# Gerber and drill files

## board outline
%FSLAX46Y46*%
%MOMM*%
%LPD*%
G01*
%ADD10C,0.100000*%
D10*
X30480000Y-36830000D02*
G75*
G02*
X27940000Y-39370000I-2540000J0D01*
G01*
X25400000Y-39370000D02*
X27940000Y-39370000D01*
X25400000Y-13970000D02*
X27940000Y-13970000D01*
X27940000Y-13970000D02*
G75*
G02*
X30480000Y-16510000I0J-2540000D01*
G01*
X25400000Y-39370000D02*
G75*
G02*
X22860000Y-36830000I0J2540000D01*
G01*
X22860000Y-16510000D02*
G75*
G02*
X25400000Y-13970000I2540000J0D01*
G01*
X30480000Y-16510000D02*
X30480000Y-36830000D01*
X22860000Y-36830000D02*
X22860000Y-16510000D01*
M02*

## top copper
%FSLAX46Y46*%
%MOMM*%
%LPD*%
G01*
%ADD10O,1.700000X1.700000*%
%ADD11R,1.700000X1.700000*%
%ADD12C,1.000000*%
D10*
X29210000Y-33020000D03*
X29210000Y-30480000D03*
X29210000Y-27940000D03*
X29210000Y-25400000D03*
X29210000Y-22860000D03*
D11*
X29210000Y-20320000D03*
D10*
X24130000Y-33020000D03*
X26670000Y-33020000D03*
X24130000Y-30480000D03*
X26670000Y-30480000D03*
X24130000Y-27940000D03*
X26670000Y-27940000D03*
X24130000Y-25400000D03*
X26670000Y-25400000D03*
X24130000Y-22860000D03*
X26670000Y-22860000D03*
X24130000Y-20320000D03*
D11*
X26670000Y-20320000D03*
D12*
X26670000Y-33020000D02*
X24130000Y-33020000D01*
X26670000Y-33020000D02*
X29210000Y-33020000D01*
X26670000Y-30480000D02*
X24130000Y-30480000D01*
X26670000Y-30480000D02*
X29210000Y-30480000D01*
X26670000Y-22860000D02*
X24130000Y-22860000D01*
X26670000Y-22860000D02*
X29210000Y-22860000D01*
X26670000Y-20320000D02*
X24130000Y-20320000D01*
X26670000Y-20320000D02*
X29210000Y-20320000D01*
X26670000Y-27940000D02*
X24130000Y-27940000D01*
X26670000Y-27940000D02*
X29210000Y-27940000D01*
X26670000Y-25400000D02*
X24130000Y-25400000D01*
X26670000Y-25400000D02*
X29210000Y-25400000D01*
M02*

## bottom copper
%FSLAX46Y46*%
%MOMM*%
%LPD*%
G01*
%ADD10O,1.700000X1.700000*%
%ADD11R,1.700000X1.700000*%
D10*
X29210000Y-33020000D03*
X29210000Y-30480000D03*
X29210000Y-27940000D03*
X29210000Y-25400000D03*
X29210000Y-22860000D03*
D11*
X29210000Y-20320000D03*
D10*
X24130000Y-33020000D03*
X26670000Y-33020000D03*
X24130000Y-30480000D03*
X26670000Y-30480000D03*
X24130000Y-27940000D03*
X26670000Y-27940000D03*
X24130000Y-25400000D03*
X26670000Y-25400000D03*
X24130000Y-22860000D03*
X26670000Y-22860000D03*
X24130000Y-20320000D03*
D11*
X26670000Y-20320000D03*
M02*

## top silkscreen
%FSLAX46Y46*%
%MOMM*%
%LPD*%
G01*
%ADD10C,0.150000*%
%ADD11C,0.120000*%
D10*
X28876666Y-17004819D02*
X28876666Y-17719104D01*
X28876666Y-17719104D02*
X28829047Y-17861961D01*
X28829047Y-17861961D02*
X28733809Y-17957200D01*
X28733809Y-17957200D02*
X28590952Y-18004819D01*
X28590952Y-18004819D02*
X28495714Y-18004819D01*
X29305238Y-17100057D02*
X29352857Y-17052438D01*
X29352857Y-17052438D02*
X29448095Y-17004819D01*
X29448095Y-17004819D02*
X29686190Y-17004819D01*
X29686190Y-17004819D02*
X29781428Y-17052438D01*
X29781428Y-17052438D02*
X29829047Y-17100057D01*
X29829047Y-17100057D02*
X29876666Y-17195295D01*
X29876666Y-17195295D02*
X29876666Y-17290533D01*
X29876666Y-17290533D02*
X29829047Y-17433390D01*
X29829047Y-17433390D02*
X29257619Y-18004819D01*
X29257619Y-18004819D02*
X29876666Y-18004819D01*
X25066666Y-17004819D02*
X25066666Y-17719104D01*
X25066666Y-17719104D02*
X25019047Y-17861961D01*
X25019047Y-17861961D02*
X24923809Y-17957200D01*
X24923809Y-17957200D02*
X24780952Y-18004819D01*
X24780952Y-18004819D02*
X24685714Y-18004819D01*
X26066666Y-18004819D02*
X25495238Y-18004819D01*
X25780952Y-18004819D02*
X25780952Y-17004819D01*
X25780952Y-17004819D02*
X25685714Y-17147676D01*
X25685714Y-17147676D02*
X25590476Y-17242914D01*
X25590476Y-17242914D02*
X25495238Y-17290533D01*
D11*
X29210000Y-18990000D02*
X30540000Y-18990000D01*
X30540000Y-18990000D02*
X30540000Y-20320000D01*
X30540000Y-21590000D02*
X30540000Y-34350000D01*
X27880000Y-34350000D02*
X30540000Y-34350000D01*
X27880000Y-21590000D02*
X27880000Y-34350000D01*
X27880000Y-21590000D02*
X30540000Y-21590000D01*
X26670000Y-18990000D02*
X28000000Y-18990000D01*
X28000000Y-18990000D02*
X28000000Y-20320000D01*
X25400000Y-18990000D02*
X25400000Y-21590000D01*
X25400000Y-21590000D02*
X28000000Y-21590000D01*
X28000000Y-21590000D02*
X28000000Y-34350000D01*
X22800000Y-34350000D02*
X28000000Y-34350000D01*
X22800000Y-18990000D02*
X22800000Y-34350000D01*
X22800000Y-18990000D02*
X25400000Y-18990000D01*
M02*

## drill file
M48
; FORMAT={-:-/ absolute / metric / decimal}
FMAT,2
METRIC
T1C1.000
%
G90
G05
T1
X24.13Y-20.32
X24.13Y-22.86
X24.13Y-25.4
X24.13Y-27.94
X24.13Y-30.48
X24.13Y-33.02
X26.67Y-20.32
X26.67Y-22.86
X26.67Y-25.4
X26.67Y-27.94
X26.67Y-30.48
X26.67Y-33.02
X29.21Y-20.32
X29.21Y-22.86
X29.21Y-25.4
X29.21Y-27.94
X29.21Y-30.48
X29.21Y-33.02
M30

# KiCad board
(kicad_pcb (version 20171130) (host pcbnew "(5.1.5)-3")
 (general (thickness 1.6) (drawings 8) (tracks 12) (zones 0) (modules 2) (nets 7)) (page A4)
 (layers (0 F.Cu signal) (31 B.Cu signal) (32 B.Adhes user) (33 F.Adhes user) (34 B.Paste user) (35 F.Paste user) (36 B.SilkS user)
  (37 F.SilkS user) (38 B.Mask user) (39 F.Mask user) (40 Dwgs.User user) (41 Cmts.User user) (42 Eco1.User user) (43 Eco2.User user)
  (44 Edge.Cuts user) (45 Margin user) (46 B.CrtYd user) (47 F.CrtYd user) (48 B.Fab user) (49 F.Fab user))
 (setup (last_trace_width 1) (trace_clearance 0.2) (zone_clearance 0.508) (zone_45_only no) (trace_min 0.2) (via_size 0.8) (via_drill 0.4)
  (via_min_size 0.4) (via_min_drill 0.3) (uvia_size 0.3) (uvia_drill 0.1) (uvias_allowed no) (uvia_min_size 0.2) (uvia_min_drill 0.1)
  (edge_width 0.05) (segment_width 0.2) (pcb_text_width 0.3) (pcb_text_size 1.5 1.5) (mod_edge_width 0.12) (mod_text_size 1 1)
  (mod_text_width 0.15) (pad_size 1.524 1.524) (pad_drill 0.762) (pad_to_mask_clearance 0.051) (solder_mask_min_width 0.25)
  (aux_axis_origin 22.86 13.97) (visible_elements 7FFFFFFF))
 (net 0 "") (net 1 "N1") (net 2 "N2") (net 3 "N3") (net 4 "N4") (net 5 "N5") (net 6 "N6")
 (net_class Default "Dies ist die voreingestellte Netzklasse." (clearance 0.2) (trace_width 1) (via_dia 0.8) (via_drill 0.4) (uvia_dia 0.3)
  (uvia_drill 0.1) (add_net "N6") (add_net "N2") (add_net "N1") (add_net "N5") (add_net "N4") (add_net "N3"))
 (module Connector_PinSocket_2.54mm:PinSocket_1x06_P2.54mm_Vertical (layer F.Cu) (at 29.21 20.32)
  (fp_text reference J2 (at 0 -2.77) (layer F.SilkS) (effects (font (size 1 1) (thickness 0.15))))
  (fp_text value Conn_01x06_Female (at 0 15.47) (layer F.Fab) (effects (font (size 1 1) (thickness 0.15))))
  (fp_line (start 0 -1.33) (end 1.33 -1.33) (layer F.SilkS) (width 0.12))
  (fp_line (start 1.33 -1.33) (end 1.33 0) (layer F.SilkS) (width 0.12))
  (fp_line (start 1.33 1.27) (end 1.33 14.03) (layer F.SilkS) (width 0.12))
  (fp_line (start -1.33 14.03) (end 1.33 14.03) (layer F.SilkS) (width 0.12))
  (fp_line (start -1.33 1.27) (end -1.33 14.03) (layer F.SilkS) (width 0.12))
  (fp_line (start -1.33 1.27) (end 1.33 1.27) (layer F.SilkS) (width 0.12))
  (pad 6 thru_hole oval (at 0 12.7) (size 1.7 1.7) (drill 1) (layers *.Cu *.Mask) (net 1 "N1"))
  (pad 5 thru_hole oval (at 0 10.16) (size 1.7 1.7) (drill 1) (layers *.Cu *.Mask) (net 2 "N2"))
  (pad 4 thru_hole oval (at 0 7.62) (size 1.7 1.7) (drill 1) (layers *.Cu *.Mask) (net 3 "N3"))
  (pad 3 thru_hole oval (at 0 5.08) (size 1.7 1.7) (drill 1) (layers *.Cu *.Mask) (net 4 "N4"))
  (pad 2 thru_hole oval (at 0 2.54) (size 1.7 1.7) (drill 1) (layers *.Cu *.Mask) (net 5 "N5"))
  (pad 1 thru_hole rect (at 0 0) (size 1.7 1.7) (drill 1) (layers *.Cu *.Mask) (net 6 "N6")))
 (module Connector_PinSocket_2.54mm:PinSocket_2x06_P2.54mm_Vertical (layer F.Cu) (at 26.67 20.32)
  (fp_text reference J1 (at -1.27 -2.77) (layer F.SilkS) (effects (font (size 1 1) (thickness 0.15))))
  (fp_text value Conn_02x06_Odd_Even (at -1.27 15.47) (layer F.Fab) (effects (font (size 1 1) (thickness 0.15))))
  (fp_line (start 0 -1.33) (end 1.33 -1.33) (layer F.SilkS) (width 0.12))
  (fp_line (start 1.33 -1.33) (end 1.33 0) (layer F.SilkS) (width 0.12))
  (fp_line (start -1.27 -1.33) (end -1.27 1.27) (layer F.SilkS) (width 0.12))
  (fp_line (start -1.27 1.27) (end 1.33 1.27) (layer F.SilkS) (width 0.12))
  (fp_line (start 1.33 1.27) (end 1.33 14.03) (layer F.SilkS) (width 0.12))
  (fp_line (start -3.87 14.03) (end 1.33 14.03) (layer F.SilkS) (width 0.12))
  (fp_line (start -3.87 -1.33) (end -3.87 14.03) (layer F.SilkS) (width 0.12))
  (fp_line (start -3.87 -1.33) (end -1.27 -1.33) (layer F.SilkS) (width 0.12))
  (pad 12 thru_hole oval (at -2.54 12.7) (size 1.7 1.7) (drill 1) (layers *.Cu *.Mask) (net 1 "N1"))
  (pad 11 thru_hole oval (at 0 12.7) (size 1.7 1.7) (drill 1) (layers *.Cu *.Mask) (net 1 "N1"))
  (pad 10 thru_hole oval (at -2.54 10.16) (size 1.7 1.7) (drill 1) (layers *.Cu *.Mask) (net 2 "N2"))
  (pad 9 thru_hole oval (at 0 10.16) (size 1.7 1.7) (drill 1) (layers *.Cu *.Mask) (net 2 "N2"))
  (pad 8 thru_hole oval (at -2.54 7.62) (size 1.7 1.7) (drill 1) (layers *.Cu *.Mask) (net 3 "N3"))
  (pad 7 thru_hole oval (at 0 7.62) (size 1.7 1.7) (drill 1) (layers *.Cu *.Mask) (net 3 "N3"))
  (pad 6 thru_hole oval (at -2.54 5.08) (size 1.7 1.7) (drill 1) (layers *.Cu *.Mask) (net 4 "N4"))
  (pad 5 thru_hole oval (at 0 5.08) (size 1.7 1.7) (drill 1) (layers *.Cu *.Mask) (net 4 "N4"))
  (pad 4 thru_hole oval (at -2.54 2.54) (size 1.7 1.7) (drill 1) (layers *.Cu *.Mask) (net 5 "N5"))
  (pad 3 thru_hole oval (at 0 2.54) (size 1.7 1.7) (drill 1) (layers *.Cu *.Mask) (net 5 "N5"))
  (pad 2 thru_hole oval (at -2.54 0) (size 1.7 1.7) (drill 1) (layers *.Cu *.Mask) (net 6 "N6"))
  (pad 1 thru_hole rect (at 0 0) (size 1.7 1.7) (drill 1) (layers *.Cu *.Mask) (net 6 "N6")))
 (gr_arc (start 27.94 36.83) (end 27.94 39.37) (angle -90) (layer Edge.Cuts) (width 0.1))
 (gr_line (start 25.4 39.37) (end 27.94 39.37) (layer Edge.Cuts) (width 0.1))
 (gr_line (start 25.4 13.97) (end 27.94 13.97) (layer Edge.Cuts) (width 0.1))
 (gr_arc (start 27.94 16.51) (end 30.48 16.51) (angle -90) (layer Edge.Cuts) (width 0.1))
 (gr_arc (start 25.4 36.83) (end 22.86 36.83) (angle -90) (layer Edge.Cuts) (width 0.1))
 (gr_arc (start 25.4 16.51) (end 25.4 13.97) (angle -90) (layer Edge.Cuts) (width 0.1))
 (gr_line (start 30.48 16.51) (end 30.48 36.83) (layer Edge.Cuts) (width 0.1))
 (gr_line (start 22.86 36.83) (end 22.86 16.51) (layer Edge.Cuts) (width 0.1))
 (segment (start 26.67 33.02) (end 24.13 33.02) (width 1) (layer F.Cu) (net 1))
 (segment (start 26.67 33.02) (end 29.21 33.02) (width 1) (layer F.Cu) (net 1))
 (segment (start 26.67 30.48) (end 24.13 30.48) (width 1) (layer F.Cu) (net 2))
 (segment (start 26.67 30.48) (end 29.21 30.48) (width 1) (layer F.Cu) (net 2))
 (segment (start 26.67 22.86) (end 24.13 22.86) (width 1) (layer F.Cu) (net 5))
 (segment (start 26.67 22.86) (end 29.21 22.86) (width 1) (layer F.Cu) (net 5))
 (segment (start 26.67 20.32) (end 24.13 20.32) (width 1) (layer F.Cu) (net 6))
 (segment (start 26.67 20.32) (end 29.21 20.32) (width 1) (layer F.Cu) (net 6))
 (segment (start 26.67 27.94) (end 24.13 27.94) (width 1) (layer F.Cu) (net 3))
 (segment (start 26.67 27.94) (end 29.21 27.94) (width 1) (layer F.Cu) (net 3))
 (segment (start 26.67 25.4) (end 24.13 25.4) (width 1) (layer F.Cu) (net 4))
 (segment (start 26.67 25.4) (end 29.21 25.4) (width 1) (layer F.Cu) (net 4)))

